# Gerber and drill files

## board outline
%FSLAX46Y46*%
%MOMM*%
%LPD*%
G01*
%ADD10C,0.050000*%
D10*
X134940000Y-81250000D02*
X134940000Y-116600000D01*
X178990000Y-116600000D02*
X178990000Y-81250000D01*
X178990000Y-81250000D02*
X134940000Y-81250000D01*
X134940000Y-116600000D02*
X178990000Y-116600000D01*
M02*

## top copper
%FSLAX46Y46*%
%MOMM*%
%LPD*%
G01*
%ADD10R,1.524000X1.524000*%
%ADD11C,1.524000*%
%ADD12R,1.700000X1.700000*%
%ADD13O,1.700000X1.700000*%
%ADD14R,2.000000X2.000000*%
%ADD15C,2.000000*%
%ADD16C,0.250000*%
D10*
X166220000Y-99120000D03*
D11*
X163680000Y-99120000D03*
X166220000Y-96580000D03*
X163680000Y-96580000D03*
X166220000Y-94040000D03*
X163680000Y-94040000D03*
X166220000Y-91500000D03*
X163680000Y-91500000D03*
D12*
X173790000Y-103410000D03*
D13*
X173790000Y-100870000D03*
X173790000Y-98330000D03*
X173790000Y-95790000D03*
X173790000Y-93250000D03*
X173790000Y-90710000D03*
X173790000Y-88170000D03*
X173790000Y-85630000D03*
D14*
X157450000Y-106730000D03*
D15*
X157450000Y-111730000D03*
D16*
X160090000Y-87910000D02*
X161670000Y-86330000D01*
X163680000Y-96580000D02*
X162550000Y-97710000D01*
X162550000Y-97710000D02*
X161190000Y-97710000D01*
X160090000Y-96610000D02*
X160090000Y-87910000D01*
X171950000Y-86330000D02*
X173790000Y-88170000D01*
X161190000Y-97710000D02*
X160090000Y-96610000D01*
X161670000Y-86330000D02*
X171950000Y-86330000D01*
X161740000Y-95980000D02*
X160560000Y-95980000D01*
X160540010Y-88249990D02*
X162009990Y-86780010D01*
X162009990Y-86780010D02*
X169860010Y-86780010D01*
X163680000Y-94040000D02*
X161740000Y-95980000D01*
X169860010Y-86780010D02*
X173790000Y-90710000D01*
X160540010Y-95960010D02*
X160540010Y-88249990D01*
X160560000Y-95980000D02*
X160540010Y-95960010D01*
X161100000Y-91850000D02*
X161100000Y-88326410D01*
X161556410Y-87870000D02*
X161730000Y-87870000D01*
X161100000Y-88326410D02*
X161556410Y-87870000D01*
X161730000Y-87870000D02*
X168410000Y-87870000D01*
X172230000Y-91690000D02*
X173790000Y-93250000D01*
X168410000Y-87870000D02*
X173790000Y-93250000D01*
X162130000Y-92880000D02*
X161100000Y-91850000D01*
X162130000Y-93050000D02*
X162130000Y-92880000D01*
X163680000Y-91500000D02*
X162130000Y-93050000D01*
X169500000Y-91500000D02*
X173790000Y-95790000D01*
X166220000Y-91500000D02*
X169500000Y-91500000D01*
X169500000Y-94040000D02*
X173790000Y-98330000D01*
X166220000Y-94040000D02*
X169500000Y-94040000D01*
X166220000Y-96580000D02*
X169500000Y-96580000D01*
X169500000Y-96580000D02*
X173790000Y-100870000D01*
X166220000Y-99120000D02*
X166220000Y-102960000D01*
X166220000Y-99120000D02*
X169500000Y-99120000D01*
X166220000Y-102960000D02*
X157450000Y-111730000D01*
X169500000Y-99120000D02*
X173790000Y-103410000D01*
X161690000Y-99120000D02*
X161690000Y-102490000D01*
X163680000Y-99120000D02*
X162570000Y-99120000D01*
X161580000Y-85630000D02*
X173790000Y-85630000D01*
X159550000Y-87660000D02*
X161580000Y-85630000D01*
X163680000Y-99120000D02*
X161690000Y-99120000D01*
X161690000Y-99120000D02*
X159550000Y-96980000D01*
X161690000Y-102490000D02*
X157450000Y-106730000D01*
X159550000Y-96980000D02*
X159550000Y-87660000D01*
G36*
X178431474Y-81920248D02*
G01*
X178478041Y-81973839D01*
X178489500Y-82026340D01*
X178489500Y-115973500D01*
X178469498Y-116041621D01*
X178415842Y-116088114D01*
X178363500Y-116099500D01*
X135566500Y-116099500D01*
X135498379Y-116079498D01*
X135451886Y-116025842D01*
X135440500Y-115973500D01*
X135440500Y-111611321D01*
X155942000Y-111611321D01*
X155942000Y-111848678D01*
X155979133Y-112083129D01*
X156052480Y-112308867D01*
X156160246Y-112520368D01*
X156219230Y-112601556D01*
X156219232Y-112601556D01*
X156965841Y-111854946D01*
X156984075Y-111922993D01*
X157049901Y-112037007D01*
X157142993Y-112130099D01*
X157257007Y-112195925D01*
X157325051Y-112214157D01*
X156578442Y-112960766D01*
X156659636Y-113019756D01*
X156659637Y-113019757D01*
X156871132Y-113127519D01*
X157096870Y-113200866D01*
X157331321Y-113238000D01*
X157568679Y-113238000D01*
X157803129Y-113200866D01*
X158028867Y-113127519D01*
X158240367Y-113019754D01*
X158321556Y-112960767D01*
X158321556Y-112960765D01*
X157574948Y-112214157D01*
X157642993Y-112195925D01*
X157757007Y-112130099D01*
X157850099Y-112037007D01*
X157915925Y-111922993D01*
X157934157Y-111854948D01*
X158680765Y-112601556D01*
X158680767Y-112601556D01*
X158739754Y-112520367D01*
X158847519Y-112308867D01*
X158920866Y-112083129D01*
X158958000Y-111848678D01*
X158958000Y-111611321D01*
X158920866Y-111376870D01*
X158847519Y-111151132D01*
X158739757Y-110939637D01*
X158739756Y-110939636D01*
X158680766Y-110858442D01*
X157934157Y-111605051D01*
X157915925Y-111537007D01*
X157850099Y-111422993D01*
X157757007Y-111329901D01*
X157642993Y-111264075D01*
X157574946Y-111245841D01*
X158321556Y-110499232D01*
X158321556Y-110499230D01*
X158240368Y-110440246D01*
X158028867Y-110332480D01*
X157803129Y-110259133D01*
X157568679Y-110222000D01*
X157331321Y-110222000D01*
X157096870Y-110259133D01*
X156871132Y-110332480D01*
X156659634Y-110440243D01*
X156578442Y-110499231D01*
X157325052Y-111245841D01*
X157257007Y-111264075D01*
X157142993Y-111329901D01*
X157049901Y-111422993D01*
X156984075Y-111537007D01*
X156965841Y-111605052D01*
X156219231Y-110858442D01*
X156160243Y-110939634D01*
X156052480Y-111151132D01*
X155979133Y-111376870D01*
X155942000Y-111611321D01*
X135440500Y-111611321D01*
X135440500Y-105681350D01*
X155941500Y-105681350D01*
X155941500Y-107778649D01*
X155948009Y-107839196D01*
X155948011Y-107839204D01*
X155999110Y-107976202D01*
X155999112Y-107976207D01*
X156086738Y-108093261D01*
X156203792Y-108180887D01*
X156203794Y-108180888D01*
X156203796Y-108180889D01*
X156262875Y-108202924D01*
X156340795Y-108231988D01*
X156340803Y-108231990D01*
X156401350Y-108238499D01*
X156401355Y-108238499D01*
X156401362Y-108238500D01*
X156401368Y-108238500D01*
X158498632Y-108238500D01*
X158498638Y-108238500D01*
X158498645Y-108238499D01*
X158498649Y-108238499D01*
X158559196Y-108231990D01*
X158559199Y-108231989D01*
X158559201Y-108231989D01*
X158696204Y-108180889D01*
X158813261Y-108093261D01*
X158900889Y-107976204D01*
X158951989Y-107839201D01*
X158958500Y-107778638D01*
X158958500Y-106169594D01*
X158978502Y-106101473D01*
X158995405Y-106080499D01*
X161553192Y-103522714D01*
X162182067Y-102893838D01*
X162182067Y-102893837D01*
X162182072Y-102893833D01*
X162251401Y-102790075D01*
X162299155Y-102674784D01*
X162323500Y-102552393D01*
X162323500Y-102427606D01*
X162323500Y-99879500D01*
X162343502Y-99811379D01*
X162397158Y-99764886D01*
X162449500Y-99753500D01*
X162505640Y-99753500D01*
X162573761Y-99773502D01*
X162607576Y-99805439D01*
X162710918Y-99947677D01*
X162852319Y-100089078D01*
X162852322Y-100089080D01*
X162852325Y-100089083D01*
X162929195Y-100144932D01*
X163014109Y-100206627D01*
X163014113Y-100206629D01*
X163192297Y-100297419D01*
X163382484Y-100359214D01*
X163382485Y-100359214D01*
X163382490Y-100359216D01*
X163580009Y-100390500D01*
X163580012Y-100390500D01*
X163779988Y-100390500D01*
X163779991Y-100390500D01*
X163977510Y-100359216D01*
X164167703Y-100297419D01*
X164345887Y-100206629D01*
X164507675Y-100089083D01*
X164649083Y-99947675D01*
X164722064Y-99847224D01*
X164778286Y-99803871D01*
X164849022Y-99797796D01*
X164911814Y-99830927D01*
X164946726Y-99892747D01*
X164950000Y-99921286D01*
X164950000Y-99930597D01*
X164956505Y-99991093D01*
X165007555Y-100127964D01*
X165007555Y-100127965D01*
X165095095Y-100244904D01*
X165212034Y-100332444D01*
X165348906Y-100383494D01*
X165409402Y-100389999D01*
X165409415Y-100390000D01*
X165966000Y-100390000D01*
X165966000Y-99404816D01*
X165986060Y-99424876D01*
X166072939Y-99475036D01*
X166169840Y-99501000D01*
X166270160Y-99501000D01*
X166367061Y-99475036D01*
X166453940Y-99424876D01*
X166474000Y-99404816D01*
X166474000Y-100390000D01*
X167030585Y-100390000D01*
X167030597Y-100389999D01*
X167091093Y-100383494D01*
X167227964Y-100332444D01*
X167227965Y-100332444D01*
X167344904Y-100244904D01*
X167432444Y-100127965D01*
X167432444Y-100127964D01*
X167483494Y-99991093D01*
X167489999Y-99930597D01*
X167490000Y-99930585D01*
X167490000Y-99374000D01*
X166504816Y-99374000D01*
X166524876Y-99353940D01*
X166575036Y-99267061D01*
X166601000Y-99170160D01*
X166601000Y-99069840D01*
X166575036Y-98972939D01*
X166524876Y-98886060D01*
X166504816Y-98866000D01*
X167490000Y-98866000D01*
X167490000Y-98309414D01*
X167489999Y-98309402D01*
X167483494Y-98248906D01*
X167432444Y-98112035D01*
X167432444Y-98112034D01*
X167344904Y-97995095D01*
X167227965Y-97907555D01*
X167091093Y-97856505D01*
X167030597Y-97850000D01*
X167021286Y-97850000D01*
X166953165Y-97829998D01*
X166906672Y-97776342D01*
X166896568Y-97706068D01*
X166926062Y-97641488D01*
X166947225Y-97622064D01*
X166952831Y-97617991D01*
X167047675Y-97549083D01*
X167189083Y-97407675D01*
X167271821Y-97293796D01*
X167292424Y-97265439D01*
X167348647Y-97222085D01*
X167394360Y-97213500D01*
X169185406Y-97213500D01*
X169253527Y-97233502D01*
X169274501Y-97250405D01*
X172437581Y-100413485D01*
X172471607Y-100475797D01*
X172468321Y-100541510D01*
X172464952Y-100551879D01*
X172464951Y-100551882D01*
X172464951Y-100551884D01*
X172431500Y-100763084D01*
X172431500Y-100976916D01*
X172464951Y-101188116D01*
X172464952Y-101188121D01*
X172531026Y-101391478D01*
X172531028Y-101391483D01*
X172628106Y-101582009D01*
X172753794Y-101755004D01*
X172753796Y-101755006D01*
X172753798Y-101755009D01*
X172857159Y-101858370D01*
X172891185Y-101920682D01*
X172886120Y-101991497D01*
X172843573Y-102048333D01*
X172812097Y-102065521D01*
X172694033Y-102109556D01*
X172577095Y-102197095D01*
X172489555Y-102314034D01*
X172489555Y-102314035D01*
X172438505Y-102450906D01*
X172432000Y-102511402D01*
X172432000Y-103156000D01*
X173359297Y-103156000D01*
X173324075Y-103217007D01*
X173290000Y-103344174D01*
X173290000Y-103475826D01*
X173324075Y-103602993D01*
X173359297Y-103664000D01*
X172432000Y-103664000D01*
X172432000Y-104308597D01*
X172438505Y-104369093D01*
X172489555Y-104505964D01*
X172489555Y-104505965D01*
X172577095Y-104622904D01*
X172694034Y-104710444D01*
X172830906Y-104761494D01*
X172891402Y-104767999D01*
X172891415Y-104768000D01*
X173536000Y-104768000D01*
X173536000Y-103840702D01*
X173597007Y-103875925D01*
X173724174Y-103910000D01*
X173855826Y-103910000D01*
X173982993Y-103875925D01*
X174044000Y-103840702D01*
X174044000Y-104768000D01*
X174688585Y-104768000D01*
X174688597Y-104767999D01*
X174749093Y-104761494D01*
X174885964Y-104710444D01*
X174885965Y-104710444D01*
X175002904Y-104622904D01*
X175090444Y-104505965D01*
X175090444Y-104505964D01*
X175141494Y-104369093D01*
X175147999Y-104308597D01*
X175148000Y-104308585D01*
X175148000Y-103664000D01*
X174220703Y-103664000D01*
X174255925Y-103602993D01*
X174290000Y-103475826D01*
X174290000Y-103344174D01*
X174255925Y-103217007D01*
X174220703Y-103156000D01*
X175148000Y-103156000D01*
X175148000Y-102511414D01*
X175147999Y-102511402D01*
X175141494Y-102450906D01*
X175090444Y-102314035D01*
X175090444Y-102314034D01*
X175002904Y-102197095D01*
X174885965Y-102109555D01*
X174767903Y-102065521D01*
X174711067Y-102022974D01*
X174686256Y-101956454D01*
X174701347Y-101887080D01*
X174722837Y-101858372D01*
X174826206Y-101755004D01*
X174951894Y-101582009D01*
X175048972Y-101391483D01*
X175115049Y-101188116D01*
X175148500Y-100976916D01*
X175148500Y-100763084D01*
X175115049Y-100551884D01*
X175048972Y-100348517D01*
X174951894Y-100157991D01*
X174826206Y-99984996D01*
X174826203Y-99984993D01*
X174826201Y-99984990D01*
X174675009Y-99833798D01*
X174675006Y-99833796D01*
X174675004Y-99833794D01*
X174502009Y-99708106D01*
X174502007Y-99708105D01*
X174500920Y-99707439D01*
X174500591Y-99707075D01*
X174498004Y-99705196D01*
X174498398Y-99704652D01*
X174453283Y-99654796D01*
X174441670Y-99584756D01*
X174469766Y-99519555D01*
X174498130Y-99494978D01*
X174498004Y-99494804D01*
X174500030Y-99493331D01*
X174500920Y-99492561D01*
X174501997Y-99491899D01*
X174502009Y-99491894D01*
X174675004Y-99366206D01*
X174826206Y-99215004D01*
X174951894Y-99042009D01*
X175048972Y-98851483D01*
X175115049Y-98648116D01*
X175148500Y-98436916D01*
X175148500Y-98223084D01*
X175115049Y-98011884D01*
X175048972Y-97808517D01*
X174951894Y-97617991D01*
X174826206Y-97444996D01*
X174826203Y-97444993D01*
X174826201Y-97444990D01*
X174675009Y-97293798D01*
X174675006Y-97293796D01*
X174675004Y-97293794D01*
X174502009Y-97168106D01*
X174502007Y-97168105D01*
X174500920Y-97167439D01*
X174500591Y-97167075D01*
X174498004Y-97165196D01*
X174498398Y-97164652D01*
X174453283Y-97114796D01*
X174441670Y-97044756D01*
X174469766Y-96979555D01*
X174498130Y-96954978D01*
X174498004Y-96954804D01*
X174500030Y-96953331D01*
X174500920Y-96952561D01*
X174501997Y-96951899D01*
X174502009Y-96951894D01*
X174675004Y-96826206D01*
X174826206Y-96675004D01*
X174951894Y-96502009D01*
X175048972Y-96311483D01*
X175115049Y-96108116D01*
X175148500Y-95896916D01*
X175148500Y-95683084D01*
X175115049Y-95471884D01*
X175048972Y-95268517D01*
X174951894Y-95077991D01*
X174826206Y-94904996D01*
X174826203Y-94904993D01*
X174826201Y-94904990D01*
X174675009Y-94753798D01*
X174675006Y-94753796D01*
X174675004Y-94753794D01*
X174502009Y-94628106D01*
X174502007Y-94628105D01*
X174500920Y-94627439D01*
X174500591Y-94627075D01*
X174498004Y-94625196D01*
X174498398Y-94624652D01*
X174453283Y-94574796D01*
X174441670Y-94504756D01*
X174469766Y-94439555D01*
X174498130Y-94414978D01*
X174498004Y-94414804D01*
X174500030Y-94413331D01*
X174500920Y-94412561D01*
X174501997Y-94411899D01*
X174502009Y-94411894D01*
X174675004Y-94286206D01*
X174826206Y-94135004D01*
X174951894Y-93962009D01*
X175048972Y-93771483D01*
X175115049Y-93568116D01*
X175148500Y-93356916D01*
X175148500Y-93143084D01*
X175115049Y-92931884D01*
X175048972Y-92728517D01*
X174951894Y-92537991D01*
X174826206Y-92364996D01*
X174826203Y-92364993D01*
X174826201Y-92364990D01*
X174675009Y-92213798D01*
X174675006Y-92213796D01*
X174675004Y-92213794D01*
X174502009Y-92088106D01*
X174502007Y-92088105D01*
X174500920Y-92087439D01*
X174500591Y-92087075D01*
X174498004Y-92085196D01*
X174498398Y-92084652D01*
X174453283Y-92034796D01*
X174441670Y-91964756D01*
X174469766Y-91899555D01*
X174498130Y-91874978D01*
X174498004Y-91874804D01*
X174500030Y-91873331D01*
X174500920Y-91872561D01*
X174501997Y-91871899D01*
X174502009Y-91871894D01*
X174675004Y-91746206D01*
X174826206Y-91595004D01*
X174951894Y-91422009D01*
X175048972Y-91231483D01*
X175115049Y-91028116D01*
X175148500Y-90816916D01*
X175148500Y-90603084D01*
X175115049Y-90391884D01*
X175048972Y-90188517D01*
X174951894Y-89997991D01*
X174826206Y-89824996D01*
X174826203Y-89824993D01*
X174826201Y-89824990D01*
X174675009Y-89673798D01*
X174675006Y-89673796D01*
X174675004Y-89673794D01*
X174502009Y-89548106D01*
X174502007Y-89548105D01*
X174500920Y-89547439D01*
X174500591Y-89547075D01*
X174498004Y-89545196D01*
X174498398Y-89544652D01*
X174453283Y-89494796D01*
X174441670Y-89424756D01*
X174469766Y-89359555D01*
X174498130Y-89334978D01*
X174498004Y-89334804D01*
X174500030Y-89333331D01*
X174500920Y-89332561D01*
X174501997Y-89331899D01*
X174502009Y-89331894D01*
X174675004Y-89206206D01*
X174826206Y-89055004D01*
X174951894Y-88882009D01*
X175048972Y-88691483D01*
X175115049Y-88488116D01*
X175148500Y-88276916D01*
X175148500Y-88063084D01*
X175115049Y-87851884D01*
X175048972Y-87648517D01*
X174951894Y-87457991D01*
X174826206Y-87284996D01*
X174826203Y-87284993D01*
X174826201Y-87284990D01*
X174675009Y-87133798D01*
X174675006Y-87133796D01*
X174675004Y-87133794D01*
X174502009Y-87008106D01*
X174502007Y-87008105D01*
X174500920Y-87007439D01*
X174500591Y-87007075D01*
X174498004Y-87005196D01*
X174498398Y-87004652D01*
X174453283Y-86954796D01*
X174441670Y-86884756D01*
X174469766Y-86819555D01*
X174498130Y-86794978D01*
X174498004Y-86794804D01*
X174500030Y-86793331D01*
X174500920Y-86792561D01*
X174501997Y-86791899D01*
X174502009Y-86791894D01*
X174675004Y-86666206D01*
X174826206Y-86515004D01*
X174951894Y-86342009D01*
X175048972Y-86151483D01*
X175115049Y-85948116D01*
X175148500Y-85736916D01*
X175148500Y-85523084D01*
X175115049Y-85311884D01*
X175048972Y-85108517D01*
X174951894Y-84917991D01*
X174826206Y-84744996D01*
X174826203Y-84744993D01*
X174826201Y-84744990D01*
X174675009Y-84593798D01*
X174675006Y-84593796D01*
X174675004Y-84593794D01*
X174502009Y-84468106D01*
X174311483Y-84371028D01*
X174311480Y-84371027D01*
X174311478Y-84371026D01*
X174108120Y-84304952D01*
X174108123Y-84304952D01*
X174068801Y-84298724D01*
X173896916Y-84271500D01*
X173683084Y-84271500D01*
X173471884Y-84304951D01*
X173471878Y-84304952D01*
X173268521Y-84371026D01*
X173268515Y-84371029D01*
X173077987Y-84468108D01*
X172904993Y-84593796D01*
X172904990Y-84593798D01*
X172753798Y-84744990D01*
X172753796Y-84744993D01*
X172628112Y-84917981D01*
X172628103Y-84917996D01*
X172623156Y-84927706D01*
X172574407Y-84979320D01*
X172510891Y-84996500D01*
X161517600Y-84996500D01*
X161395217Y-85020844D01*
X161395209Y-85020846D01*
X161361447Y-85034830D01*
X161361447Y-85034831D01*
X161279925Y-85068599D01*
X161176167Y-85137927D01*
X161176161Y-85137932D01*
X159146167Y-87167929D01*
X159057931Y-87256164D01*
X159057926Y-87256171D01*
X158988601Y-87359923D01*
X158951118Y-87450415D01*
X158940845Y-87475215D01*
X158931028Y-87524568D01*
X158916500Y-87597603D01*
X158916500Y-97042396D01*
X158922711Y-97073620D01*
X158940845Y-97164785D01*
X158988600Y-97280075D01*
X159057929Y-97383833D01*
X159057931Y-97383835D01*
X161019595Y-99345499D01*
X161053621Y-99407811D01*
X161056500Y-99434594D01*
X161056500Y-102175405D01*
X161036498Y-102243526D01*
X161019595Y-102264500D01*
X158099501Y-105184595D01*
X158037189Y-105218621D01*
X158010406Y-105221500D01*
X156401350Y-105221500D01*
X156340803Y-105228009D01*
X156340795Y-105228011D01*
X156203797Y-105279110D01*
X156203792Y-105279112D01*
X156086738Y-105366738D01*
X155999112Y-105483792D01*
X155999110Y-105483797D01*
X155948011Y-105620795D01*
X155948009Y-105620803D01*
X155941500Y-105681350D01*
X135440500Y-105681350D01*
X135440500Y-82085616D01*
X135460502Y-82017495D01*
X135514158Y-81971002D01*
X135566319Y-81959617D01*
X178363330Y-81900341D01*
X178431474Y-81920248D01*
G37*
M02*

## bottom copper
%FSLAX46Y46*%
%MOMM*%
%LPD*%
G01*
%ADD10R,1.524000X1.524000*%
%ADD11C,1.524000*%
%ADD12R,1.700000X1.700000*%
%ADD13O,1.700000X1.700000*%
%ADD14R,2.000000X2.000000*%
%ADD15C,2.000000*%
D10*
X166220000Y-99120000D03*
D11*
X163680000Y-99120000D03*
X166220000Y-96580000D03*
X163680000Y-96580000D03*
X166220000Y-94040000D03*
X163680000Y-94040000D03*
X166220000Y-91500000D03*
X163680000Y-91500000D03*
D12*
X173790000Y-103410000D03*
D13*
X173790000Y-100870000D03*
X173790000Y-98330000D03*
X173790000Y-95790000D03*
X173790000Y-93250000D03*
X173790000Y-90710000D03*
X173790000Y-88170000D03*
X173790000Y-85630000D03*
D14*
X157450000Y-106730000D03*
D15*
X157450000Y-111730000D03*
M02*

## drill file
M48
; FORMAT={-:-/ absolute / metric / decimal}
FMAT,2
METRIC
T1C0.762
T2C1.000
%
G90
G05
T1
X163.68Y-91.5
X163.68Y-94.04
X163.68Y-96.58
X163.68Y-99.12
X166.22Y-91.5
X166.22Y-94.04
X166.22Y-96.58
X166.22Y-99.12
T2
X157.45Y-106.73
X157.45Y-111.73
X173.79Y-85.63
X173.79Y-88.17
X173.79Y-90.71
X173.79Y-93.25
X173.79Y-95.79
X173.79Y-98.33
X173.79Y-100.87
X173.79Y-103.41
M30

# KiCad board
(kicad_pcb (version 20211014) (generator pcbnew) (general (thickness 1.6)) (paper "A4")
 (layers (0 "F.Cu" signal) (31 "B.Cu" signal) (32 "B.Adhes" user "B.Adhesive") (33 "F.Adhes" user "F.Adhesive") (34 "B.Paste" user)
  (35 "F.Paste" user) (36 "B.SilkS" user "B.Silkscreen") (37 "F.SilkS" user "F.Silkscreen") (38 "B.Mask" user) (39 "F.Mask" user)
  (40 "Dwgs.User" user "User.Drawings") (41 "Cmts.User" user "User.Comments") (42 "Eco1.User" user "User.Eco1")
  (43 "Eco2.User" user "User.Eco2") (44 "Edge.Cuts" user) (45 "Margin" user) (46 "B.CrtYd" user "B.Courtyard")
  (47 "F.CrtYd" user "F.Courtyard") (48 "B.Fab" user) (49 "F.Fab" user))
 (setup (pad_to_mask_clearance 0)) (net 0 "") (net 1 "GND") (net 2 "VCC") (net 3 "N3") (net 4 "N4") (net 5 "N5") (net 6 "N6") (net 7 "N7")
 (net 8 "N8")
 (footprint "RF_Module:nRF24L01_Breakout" (layer "F.Cu") (at 166.22 99.12 180)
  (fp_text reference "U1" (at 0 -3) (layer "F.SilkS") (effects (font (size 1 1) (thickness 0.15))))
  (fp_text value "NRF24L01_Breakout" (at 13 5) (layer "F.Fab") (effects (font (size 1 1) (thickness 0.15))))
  (pad "1" thru_hole rect locked (at 0 0 180) (size 1.524 1.524) (drill 0.762) (layers *.Cu *.Mask) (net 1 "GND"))
  (pad "2" thru_hole circle locked (at 2.54 0 180) (size 1.524 1.524) (drill 0.762) (layers *.Cu *.Mask) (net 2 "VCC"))
  (pad "3" thru_hole circle locked (at 0 2.54 180) (size 1.524 1.524) (drill 0.762) (layers *.Cu *.Mask) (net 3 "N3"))
  (pad "4" thru_hole circle locked (at 2.54 2.54 180) (size 1.524 1.524) (drill 0.762) (layers *.Cu *.Mask) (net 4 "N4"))
  (pad "5" thru_hole circle locked (at 0 5.08 180) (size 1.524 1.524) (drill 0.762) (layers *.Cu *.Mask) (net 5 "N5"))
  (pad "6" thru_hole circle locked (at 2.54 5.08 180) (size 1.524 1.524) (drill 0.762) (layers *.Cu *.Mask) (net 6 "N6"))
  (pad "7" thru_hole circle locked (at 0 7.62 180) (size 1.524 1.524) (drill 0.762) (layers *.Cu *.Mask) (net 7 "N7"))
  (pad "8" thru_hole circle locked (at 2.54 7.62 180) (size 1.524 1.524) (drill 0.762) (layers *.Cu *.Mask) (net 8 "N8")))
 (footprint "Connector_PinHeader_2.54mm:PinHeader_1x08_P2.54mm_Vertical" (layer "F.Cu") (at 173.79 103.41 180)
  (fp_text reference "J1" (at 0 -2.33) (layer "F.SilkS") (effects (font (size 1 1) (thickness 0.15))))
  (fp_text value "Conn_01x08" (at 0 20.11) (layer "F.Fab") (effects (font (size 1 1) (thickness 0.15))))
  (pad "1" thru_hole rect locked (at 0 0 180) (size 1.7 1.7) (drill 1) (layers *.Cu *.Mask) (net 1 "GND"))
  (pad "2" thru_hole oval locked (at 0 2.54 180) (size 1.7 1.7) (drill 1) (layers *.Cu *.Mask) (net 3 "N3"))
  (pad "3" thru_hole oval locked (at 0 5.08 180) (size 1.7 1.7) (drill 1) (layers *.Cu *.Mask) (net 5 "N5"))
  (pad "4" thru_hole oval locked (at 0 7.62 180) (size 1.7 1.7) (drill 1) (layers *.Cu *.Mask) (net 7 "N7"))
  (pad "5" thru_hole oval locked (at 0 10.16 180) (size 1.7 1.7) (drill 1) (layers *.Cu *.Mask) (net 8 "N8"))
  (pad "6" thru_hole oval locked (at 0 12.7 180) (size 1.7 1.7) (drill 1) (layers *.Cu *.Mask) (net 6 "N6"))
  (pad "7" thru_hole oval locked (at 0 15.24 180) (size 1.7 1.7) (drill 1) (layers *.Cu *.Mask) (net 4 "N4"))
  (pad "8" thru_hole oval locked (at 0 17.78 180) (size 1.7 1.7) (drill 1) (layers *.Cu *.Mask) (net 2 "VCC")))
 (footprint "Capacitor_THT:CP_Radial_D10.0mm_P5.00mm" (layer "F.Cu") (at 157.45 106.73 -90)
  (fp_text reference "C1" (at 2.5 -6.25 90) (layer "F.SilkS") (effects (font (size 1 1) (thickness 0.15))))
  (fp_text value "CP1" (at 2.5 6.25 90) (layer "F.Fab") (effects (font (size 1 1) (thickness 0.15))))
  (pad "1" thru_hole rect locked (at 0 0 270) (size 2 2) (drill 1) (layers *.Cu *.Mask) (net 2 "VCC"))
  (pad "2" thru_hole circle locked (at 5 0 270) (size 2 2) (drill 1) (layers *.Cu *.Mask) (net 1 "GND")))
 (gr_line (start 134.94 81.25) (end 134.94 116.6) (layer "Edge.Cuts") (width 0.05))
 (gr_line (start 178.99 116.6) (end 178.99 81.25) (layer "Edge.Cuts") (width 0.05))
 (gr_line (start 178.99 81.25) (end 134.94 81.25) (layer "Edge.Cuts") (width 0.05))
 (gr_line (start 134.94 116.6) (end 178.99 116.6) (layer "Edge.Cuts") (width 0.05))
 (segment (start 160.09 87.91) (end 161.67 86.33) (width 0.25) (layer "F.Cu") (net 4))
 (segment (start 163.68 96.58) (end 162.55 97.71) (width 0.25) (layer "F.Cu") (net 4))
 (segment (start 162.55 97.71) (end 161.19 97.71) (width 0.25) (layer "F.Cu") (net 4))
 (segment (start 160.09 96.61) (end 160.09 87.91) (width 0.25) (layer "F.Cu") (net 4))
 (segment (start 171.95 86.33) (end 173.79 88.17) (width 0.25) (layer "F.Cu") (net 4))
 (segment (start 161.19 97.71) (end 160.09 96.61) (width 0.25) (layer "F.Cu") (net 4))
 (segment (start 161.67 86.33) (end 171.95 86.33) (width 0.25) (layer "F.Cu") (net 4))
 (segment (start 161.74 95.98) (end 160.56 95.98) (width 0.25) (layer "F.Cu") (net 6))
 (segment (start 160.54001 88.24999) (end 162.00999 86.78001) (width 0.25) (layer "F.Cu") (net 6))
 (segment (start 162.00999 86.78001) (end 169.86001 86.78001) (width 0.25) (layer "F.Cu") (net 6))
 (segment (start 163.68 94.04) (end 161.74 95.98) (width 0.25) (layer "F.Cu") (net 6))
 (segment (start 169.86001 86.78001) (end 173.79 90.71) (width 0.25) (layer "F.Cu") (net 6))
 (segment (start 160.54001 95.96001) (end 160.54001 88.24999) (width 0.25) (layer "F.Cu") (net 6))
 (segment (start 160.56 95.98) (end 160.54001 95.96001) (width 0.25) (layer "F.Cu") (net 6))
 (segment (start 161.1 91.85) (end 161.1 88.32641) (width 0.25) (layer "F.Cu") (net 8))
 (segment (start 161.55641 87.87) (end 161.73 87.87) (width 0.25) (layer "F.Cu") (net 8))
 (segment (start 161.1 88.32641) (end 161.55641 87.87) (width 0.25) (layer "F.Cu") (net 8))
 (segment (start 161.73 87.87) (end 168.41 87.87) (width 0.25) (layer "F.Cu") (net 8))
 (segment (start 172.23 91.69) (end 173.79 93.25) (width 0.25) (layer "F.Cu") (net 8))
 (segment (start 168.41 87.87) (end 173.79 93.25) (width 0.25) (layer "F.Cu") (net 8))
 (segment (start 162.13 92.88) (end 161.1 91.85) (width 0.25) (layer "F.Cu") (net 8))
 (segment (start 162.13 93.05) (end 162.13 92.88) (width 0.25) (layer "F.Cu") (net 8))
 (segment (start 163.68 91.5) (end 162.13 93.05) (width 0.25) (layer "F.Cu") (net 8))
 (segment (start 169.5 91.5) (end 173.79 95.79) (width 0.25) (layer "F.Cu") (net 7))
 (segment (start 166.22 91.5) (end 169.5 91.5) (width 0.25) (layer "F.Cu") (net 7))
 (segment (start 169.5 94.04) (end 173.79 98.33) (width 0.25) (layer "F.Cu") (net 5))
 (segment (start 166.22 94.04) (end 169.5 94.04) (width 0.25) (layer "F.Cu") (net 5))
 (segment (start 166.22 96.58) (end 169.5 96.58) (width 0.25) (layer "F.Cu") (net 3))
 (segment (start 169.5 96.58) (end 173.79 100.87) (width 0.25) (layer "F.Cu") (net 3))
 (segment (start 166.22 99.12) (end 166.22 102.96) (width 0.25) (layer "F.Cu") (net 1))
 (segment (start 166.22 99.12) (end 169.5 99.12) (width 0.25) (layer "F.Cu") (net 1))
 (segment (start 166.22 102.96) (end 157.45 111.73) (width 0.25) (layer "F.Cu") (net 1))
 (segment (start 169.5 99.12) (end 173.79 103.41) (width 0.25) (layer "F.Cu") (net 1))
 (segment (start 161.69 99.12) (end 161.69 102.49) (width 0.25) (layer "F.Cu") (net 2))
 (segment (start 163.68 99.12) (end 162.57 99.12) (width 0.25) (layer "F.Cu") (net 2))
 (segment (start 161.58 85.63) (end 173.79 85.63) (width 0.25) (layer "F.Cu") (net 2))
 (segment (start 159.55 87.66) (end 161.58 85.63) (width 0.25) (layer "F.Cu") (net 2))
 (segment (start 163.68 99.12) (end 161.69 99.12) (width 0.25) (layer "F.Cu") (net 2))
 (segment (start 161.69 99.12) (end 159.55 96.98) (width 0.25) (layer "F.Cu") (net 2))
 (segment (start 161.69 102.49) (end 157.45 106.73) (width 0.25) (layer "F.Cu") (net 2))
 (segment (start 159.55 96.98) (end 159.55 87.66) (width 0.25) (layer "F.Cu") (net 2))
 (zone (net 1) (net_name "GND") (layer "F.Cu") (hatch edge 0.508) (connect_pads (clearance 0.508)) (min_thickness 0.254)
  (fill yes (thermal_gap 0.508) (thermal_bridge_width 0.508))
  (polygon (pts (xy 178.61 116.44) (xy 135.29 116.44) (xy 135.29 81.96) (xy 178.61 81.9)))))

